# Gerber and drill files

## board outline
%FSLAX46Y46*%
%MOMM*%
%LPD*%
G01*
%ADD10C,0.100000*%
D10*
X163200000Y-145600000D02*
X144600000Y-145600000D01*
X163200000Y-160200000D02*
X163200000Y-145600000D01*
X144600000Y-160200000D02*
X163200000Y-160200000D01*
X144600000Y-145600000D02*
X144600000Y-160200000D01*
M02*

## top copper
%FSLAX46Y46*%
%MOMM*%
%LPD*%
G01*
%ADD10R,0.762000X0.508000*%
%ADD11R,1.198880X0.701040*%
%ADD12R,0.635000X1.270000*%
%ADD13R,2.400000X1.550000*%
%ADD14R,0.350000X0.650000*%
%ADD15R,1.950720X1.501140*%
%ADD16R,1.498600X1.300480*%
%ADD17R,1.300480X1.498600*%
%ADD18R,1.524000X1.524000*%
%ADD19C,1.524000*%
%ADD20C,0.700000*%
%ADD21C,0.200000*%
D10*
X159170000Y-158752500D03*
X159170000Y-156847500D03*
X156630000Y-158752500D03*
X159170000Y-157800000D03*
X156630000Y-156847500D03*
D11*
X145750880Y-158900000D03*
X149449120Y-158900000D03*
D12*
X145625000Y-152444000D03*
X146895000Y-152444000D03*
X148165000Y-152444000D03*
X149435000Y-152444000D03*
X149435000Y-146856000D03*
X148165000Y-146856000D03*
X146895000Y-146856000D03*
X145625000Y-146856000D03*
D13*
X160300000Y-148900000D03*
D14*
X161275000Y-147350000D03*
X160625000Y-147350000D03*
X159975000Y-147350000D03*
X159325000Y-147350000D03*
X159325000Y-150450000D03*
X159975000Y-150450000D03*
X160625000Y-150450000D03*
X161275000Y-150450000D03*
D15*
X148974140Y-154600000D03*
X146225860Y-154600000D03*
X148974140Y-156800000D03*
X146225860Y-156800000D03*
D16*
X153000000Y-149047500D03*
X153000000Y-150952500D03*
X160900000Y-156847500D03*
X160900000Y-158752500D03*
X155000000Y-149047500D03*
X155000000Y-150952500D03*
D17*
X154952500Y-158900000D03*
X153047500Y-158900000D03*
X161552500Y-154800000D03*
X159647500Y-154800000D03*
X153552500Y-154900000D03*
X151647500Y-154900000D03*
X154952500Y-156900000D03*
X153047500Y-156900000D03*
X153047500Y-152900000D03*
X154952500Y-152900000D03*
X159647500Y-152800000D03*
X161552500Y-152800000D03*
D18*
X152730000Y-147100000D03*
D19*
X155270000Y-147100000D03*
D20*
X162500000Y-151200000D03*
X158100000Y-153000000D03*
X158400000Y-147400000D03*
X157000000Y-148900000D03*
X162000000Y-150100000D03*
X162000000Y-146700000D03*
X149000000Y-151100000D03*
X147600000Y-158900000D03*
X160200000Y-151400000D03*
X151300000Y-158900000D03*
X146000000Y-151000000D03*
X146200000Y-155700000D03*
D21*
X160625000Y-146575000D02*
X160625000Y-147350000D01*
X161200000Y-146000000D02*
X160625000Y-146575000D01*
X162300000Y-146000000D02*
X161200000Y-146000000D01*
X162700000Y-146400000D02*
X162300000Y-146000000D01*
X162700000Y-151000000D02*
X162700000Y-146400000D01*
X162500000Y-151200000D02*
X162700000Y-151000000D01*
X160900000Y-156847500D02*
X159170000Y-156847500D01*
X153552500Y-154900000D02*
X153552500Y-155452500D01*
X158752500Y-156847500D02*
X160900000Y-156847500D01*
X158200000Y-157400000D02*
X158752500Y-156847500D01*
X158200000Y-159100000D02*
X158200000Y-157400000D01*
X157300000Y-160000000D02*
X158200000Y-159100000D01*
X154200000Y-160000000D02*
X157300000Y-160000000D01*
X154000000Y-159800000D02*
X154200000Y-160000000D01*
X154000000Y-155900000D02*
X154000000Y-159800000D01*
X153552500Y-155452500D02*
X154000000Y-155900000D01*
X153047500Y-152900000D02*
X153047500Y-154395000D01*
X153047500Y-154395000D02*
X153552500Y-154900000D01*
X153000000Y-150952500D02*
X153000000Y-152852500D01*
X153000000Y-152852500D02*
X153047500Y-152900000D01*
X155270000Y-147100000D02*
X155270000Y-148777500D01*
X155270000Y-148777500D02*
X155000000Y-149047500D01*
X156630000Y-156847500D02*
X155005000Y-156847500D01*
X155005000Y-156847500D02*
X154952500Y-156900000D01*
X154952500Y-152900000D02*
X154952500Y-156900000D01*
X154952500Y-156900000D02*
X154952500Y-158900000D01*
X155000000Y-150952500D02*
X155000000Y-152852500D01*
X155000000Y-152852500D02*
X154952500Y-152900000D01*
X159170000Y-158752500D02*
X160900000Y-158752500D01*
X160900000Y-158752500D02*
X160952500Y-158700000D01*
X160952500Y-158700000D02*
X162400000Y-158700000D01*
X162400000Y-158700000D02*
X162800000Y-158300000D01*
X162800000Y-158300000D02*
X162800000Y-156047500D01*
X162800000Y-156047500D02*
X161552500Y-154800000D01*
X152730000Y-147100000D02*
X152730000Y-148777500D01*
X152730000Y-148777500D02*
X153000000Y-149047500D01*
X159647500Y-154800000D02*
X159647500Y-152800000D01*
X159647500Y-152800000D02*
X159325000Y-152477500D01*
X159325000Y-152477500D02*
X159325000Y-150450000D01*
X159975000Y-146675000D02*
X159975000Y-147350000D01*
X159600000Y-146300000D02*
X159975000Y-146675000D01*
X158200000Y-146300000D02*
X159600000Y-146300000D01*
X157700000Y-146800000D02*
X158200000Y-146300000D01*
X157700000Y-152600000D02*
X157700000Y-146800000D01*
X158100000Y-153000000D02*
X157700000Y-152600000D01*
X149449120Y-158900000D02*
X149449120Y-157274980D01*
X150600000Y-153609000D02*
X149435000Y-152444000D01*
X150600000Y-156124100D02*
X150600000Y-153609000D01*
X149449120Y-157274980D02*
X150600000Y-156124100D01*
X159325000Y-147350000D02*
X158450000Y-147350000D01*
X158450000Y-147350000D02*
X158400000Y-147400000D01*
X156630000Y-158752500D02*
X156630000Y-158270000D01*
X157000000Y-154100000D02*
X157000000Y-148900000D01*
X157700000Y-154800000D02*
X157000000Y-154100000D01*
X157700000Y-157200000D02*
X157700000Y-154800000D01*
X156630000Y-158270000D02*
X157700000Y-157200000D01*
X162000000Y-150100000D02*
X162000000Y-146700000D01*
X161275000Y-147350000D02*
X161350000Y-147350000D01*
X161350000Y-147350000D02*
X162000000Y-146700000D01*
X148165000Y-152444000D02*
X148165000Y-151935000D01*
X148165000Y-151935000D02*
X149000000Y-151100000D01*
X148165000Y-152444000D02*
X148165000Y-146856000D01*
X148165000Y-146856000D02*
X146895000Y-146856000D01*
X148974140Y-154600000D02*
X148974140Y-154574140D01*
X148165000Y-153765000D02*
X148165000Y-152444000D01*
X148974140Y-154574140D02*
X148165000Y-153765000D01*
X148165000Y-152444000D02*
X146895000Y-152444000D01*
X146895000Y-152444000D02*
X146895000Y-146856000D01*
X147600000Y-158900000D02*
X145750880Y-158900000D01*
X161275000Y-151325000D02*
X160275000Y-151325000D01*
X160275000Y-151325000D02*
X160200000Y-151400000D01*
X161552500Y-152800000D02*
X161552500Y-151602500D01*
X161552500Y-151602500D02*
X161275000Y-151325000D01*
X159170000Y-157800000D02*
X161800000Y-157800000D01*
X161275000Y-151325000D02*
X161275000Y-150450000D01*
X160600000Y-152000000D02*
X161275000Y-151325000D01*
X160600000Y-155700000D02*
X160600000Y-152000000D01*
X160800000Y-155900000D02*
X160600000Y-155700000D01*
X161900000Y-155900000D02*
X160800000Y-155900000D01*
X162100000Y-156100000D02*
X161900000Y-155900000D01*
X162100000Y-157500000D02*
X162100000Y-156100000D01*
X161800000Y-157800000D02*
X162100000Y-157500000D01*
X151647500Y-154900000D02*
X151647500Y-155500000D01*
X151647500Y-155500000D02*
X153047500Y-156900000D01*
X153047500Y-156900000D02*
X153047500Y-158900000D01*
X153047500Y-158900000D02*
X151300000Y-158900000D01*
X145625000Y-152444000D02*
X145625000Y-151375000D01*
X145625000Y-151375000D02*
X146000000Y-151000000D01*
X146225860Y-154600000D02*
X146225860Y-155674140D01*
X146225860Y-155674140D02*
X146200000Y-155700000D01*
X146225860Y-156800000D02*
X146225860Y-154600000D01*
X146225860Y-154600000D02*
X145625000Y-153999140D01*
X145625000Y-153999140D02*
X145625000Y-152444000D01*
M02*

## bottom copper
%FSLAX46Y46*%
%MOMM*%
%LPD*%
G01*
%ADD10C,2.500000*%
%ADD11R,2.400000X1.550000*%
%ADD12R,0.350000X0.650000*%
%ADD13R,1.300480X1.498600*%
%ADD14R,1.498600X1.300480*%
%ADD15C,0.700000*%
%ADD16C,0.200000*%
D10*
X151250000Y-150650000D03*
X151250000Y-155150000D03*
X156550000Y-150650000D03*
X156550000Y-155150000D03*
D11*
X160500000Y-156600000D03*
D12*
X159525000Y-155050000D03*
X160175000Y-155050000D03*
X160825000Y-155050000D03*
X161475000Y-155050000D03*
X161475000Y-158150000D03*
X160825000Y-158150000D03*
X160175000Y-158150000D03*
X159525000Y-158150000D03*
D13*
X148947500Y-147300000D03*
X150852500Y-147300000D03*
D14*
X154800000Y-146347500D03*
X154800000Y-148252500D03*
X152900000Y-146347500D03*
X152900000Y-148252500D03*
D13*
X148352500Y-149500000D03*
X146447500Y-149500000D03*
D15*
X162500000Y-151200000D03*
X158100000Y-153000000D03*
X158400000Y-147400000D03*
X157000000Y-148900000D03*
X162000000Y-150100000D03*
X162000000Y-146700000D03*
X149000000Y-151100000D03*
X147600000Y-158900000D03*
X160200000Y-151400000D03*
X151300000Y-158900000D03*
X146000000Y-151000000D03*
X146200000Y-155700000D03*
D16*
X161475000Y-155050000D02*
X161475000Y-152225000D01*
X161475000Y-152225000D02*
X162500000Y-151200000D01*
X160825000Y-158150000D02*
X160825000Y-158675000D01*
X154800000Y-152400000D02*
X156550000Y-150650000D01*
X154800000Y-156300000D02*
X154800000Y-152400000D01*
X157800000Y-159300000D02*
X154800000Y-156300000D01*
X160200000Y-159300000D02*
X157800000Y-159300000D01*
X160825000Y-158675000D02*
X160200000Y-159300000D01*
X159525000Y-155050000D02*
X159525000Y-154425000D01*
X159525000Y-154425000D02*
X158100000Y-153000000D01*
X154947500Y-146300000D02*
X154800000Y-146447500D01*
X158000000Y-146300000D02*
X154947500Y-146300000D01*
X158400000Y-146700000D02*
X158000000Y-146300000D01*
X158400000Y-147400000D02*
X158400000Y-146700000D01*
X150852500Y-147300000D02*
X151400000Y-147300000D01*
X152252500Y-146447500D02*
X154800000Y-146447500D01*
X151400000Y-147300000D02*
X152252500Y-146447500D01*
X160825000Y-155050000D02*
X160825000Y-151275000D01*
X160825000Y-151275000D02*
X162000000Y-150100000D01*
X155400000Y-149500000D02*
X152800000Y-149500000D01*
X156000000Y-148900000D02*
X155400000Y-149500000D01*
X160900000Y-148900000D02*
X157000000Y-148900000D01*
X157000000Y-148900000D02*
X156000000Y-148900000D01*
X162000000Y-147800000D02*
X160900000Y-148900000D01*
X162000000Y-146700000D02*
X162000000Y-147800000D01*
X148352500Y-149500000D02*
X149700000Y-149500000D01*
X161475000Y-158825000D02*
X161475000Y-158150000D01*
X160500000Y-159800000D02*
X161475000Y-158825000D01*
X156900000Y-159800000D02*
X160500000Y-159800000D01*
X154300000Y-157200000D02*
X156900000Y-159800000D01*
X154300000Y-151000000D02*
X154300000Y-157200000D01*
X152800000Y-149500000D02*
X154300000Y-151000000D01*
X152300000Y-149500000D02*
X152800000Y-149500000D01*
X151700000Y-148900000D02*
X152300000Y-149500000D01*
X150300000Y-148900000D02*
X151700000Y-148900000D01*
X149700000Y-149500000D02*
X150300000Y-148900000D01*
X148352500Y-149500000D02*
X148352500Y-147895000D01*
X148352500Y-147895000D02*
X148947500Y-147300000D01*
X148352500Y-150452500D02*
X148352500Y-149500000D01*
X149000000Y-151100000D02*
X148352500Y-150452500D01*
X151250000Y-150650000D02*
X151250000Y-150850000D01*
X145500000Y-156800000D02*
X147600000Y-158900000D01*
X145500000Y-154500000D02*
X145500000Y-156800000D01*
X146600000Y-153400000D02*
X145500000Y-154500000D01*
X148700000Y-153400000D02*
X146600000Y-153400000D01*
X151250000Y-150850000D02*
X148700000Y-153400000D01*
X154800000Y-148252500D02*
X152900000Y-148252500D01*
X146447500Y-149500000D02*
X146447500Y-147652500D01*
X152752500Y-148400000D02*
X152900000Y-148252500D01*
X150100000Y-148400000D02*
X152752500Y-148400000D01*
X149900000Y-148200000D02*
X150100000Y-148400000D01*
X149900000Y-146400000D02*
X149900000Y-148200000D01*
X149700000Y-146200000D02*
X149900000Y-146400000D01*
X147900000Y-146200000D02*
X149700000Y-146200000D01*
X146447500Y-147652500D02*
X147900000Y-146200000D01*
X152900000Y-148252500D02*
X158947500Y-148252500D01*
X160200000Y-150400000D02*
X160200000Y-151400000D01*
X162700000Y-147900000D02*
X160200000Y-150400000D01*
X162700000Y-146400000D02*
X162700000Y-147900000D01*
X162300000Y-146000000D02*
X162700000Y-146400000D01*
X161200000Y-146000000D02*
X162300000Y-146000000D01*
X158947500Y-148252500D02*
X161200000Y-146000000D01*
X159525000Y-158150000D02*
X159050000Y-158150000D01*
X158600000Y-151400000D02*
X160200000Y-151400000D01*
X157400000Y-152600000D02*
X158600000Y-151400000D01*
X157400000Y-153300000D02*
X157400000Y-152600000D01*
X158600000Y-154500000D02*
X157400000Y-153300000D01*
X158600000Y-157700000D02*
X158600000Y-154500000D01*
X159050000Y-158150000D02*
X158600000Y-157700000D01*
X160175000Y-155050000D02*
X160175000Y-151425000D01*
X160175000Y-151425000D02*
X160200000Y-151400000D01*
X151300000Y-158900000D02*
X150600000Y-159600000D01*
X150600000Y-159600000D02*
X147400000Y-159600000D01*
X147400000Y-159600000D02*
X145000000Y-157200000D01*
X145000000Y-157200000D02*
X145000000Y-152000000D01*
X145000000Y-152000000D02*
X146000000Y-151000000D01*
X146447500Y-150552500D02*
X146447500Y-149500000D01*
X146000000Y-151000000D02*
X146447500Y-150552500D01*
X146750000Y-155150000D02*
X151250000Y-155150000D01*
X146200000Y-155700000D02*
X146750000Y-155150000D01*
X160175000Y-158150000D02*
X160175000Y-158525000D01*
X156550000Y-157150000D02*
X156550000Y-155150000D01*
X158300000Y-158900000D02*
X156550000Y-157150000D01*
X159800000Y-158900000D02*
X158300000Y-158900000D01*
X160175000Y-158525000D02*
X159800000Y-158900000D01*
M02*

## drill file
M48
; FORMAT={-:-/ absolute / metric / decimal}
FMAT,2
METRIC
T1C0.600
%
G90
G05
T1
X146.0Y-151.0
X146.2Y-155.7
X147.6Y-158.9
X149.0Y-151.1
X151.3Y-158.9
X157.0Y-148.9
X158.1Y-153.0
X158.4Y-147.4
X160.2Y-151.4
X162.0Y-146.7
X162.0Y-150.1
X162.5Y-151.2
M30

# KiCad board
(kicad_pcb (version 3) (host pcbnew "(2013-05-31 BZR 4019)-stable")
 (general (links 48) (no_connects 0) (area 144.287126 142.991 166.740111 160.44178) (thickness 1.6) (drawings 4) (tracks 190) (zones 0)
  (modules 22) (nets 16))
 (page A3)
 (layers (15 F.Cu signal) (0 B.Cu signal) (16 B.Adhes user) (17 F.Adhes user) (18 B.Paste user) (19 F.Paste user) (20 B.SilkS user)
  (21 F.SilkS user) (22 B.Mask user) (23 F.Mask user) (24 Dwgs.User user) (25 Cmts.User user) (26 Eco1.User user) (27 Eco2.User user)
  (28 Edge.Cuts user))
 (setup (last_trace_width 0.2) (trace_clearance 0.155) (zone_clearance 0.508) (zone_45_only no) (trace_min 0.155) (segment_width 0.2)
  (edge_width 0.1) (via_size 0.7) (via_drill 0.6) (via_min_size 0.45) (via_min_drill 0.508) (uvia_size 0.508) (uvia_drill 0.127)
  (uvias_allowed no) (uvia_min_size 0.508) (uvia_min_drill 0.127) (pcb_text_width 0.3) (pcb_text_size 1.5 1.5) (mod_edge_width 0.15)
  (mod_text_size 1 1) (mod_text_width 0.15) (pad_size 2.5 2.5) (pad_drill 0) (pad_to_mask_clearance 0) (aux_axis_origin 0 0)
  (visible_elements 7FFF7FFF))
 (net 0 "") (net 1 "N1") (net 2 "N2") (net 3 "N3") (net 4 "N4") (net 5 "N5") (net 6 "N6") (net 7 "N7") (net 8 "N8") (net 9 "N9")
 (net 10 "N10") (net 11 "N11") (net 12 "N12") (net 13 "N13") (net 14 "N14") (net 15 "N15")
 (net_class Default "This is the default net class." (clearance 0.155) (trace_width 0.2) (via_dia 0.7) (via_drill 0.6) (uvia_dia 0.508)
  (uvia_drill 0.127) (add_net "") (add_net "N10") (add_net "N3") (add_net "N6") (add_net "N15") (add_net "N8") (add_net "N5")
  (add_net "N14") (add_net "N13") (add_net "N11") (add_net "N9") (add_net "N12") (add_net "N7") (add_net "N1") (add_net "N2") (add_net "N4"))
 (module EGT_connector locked (layer B.Cu) (at 153.9 152.9)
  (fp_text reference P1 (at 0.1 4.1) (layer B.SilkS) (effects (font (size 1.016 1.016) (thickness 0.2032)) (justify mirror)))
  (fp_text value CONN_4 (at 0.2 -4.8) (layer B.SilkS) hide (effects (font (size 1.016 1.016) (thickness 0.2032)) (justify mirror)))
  (pad 1 smd circle (at -2.65 -2.25) (size 2.5 2.5) (layers B.Cu B.Paste B.Mask) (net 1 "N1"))
  (pad 2 smd circle (at -2.65 2.25) (size 2.5 2.5) (layers B.Cu B.Paste B.Mask) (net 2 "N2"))
  (pad 3 smd circle (at 2.65 -2.25) (size 2.5 2.5) (layers B.Cu B.Paste B.Mask) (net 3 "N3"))
  (pad 4 smd circle (at 2.65 2.25) (size 2.5 2.5) (layers B.Cu B.Paste B.Mask) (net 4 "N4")))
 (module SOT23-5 (layer F.Cu) (at 157.9 157.8 90)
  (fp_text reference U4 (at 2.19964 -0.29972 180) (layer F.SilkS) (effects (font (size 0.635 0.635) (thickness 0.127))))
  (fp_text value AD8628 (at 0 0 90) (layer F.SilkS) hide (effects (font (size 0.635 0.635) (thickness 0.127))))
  (pad 1 smd rect (at -0.9525 1.27 90) (size 0.508 0.762) (layers F.Cu F.Paste F.Mask) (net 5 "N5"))
  (pad 3 smd rect (at 0.9525 1.27 90) (size 0.508 0.762) (layers F.Cu F.Paste F.Mask) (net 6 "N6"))
  (pad 5 smd rect (at -0.9525 -1.27 90) (size 0.508 0.762) (layers F.Cu F.Paste F.Mask) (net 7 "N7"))
  (pad 2 smd rect (at 0 1.27 90) (size 0.508 0.762) (layers F.Cu F.Paste F.Mask) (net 2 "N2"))
  (pad 4 smd rect (at 0.9525 -1.27 90) (size 0.508 0.762) (layers F.Cu F.Paste F.Mask) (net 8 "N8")))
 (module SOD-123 (layer F.Cu) (at 147.6 158.9)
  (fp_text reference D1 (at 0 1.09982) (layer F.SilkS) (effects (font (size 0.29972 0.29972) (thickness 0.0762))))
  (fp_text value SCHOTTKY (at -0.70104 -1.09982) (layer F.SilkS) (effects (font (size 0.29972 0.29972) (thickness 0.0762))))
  (pad 1 smd rect (at -1.84912 0) (size 1.19888 0.70104) (layers F.Cu F.Paste F.Mask) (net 1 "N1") (clearance 0.14986))
  (pad 2 smd rect (at 1.84912 0) (size 1.19888 0.70104) (layers F.Cu F.Paste F.Mask) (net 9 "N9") (clearance 0.14986)))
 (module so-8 (layer F.Cu) (at 147.53 149.65)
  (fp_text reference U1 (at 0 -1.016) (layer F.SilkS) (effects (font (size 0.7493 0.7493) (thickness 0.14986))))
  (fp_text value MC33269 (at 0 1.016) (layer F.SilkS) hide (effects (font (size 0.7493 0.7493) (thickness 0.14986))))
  (pad 1 smd rect (at -1.905 2.794) (size 0.635 1.27) (layers F.Cu F.Paste F.Mask) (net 2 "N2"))
  (pad 2 smd rect (at -0.635 2.794) (size 0.635 1.27) (layers F.Cu F.Paste F.Mask) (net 7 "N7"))
  (pad 3 smd rect (at 0.635 2.794) (size 0.635 1.27) (layers F.Cu F.Paste F.Mask) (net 7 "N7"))
  (pad 4 smd rect (at 1.905 2.794) (size 0.635 1.27) (layers F.Cu F.Paste F.Mask) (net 9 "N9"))
  (pad 5 smd rect (at 1.905 -2.794) (size 0.635 1.27) (layers F.Cu F.Paste F.Mask))
  (pad 6 smd rect (at 0.635 -2.794) (size 0.635 1.27) (layers F.Cu F.Paste F.Mask) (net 7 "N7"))
  (pad 7 smd rect (at -0.635 -2.794) (size 0.635 1.27) (layers F.Cu F.Paste F.Mask) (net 7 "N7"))
  (pad 8 smd rect (at -1.905 -2.794) (size 0.635 1.27) (layers F.Cu F.Paste F.Mask)))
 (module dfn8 (layer F.Cu) (at 160.3 148.9 180)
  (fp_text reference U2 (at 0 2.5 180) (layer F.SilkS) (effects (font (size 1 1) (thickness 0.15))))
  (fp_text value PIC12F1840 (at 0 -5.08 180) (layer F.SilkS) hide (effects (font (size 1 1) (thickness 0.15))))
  (pad 9 smd rect (at 0 0 180) (size 2.4 1.55) (layers F.Cu F.Paste F.Mask))
  (pad 1 smd rect (at -0.975 1.55 180) (size 0.35 0.65) (layers F.Cu F.Paste F.Mask) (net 7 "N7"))
  (pad 2 smd rect (at -0.325 1.55 180) (size 0.35 0.65) (layers F.Cu F.Paste F.Mask) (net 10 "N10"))
  (pad 3 smd rect (at 0.325 1.55 180) (size 0.35 0.65) (layers F.Cu F.Paste F.Mask) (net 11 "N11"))
  (pad 4 smd rect (at 0.975 1.55 180) (size 0.35 0.65) (layers F.Cu F.Paste F.Mask) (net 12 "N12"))
  (pad 5 smd rect (at 0.975 -1.55 180) (size 0.35 0.65) (layers F.Cu F.Paste F.Mask) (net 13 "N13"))
  (pad 6 smd rect (at 0.325 -1.55 180) (size 0.35 0.65) (layers F.Cu F.Paste F.Mask))
  (pad 7 smd rect (at -0.325 -1.55 180) (size 0.35 0.65) (layers F.Cu F.Paste F.Mask))
  (pad 8 smd rect (at -0.975 -1.55 180) (size 0.35 0.65) (layers F.Cu F.Paste F.Mask) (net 2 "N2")))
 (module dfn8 (layer B.Cu) (at 160.5 156.6)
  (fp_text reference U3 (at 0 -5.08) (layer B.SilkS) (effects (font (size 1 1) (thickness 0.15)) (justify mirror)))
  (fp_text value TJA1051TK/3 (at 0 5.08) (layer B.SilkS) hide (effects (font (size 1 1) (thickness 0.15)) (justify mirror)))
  (pad 9 smd rect (at 0 0) (size 2.4 1.55) (layers B.Cu B.Paste B.Mask))
  (pad 1 smd rect (at -0.975 -1.55) (size 0.35 0.65) (layers B.Cu B.Paste B.Mask) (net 11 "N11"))
  (pad 2 smd rect (at -0.325 -1.55) (size 0.35 0.65) (layers B.Cu B.Paste B.Mask) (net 2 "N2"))
  (pad 3 smd rect (at 0.325 -1.55) (size 0.35 0.65) (layers B.Cu B.Paste B.Mask) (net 7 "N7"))
  (pad 4 smd rect (at 0.975 -1.55) (size 0.35 0.65) (layers B.Cu B.Paste B.Mask) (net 10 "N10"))
  (pad 5 smd rect (at 0.975 1.55) (size 0.35 0.65) (layers B.Cu B.Paste B.Mask) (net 7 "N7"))
  (pad 6 smd rect (at 0.325 1.55) (size 0.35 0.65) (layers B.Cu B.Paste B.Mask) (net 3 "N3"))
  (pad 7 smd rect (at -0.325 1.55) (size 0.35 0.65) (layers B.Cu B.Paste B.Mask) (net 4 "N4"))
  (pad 8 smd rect (at -0.975 1.55) (size 0.35 0.65) (layers B.Cu B.Paste B.Mask) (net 2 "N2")))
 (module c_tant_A (layer F.Cu) (at 147.6 154.6)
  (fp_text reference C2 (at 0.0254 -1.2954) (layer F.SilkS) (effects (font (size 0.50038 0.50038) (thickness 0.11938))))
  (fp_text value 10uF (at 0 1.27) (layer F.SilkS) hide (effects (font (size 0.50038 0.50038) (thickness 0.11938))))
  (pad 1 smd rect (at 1.37414 0) (size 1.95072 1.50114) (layers F.Cu F.Paste F.Mask) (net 7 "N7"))
  (pad 2 smd rect (at -1.37414 0) (size 1.95072 1.50114) (layers F.Cu F.Paste F.Mask) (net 2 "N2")))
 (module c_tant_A (layer F.Cu) (at 147.6 156.8)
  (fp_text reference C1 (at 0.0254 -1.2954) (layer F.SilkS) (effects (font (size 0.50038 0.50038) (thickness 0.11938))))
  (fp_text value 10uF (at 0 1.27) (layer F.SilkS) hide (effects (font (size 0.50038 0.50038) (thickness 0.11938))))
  (pad 1 smd rect (at 1.37414 0) (size 1.95072 1.50114) (layers F.Cu F.Paste F.Mask) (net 9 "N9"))
  (pad 2 smd rect (at -1.37414 0) (size 1.95072 1.50114) (layers F.Cu F.Paste F.Mask) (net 2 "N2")))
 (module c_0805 (layer F.Cu) (at 153 150 90)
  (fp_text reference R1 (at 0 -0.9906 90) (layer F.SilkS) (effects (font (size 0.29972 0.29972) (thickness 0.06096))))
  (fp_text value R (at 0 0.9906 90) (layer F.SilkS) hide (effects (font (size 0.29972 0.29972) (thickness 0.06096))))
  (pad 1 smd rect (at 0.9525 0 90) (size 1.30048 1.4986) (layers F.Cu F.Paste F.Mask) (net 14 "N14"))
  (pad 2 smd rect (at -0.9525 0 90) (size 1.30048 1.4986) (layers F.Cu F.Paste F.Mask) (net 6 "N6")))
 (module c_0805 (layer F.Cu) (at 160.9 157.8 90)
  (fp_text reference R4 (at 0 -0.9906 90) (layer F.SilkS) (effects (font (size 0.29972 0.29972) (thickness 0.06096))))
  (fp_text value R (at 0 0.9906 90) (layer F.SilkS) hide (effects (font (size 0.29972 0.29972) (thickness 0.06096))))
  (pad 1 smd rect (at 0.9525 0 90) (size 1.30048 1.4986) (layers F.Cu F.Paste F.Mask) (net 6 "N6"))
  (pad 2 smd rect (at -0.9525 0 90) (size 1.30048 1.4986) (layers F.Cu F.Paste F.Mask) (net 5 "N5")))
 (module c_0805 (layer F.Cu) (at 155 150 90)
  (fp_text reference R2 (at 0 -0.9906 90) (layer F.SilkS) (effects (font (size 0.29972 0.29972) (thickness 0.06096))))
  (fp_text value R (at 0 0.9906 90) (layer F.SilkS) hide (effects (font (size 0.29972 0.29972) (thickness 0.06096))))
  (pad 1 smd rect (at 0.9525 0 90) (size 1.30048 1.4986) (layers F.Cu F.Paste F.Mask) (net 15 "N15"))
  (pad 2 smd rect (at -0.9525 0 90) (size 1.30048 1.4986) (layers F.Cu F.Paste F.Mask) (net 8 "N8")))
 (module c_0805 (layer F.Cu) (at 154 158.9)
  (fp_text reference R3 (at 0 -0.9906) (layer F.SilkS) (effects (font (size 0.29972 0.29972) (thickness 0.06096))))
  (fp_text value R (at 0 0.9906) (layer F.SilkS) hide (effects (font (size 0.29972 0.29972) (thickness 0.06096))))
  (pad 1 smd rect (at 0.9525 0) (size 1.30048 1.4986) (layers F.Cu F.Paste F.Mask) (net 8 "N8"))
  (pad 2 smd rect (at -0.9525 0) (size 1.30048 1.4986) (layers F.Cu F.Paste F.Mask) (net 2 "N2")))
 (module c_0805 (layer B.Cu) (at 149.9 147.3 180)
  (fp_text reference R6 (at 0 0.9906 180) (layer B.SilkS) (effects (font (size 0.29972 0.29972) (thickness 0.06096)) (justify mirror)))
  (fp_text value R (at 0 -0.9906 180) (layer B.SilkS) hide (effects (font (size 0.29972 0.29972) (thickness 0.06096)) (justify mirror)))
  (pad 1 smd rect (at 0.9525 0 180) (size 1.30048 1.4986) (layers B.Cu B.Paste B.Mask) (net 7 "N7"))
  (pad 2 smd rect (at -0.9525 0 180) (size 1.30048 1.4986) (layers B.Cu B.Paste B.Mask) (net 12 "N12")))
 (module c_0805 (layer F.Cu) (at 160.6 154.8)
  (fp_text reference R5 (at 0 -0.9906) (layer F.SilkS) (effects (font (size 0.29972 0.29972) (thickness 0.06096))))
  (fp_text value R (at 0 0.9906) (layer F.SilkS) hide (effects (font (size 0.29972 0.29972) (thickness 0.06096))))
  (pad 1 smd rect (at 0.9525 0) (size 1.30048 1.4986) (layers F.Cu F.Paste F.Mask) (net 5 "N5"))
  (pad 2 smd rect (at -0.9525 0) (size 1.30048 1.4986) (layers F.Cu F.Paste F.Mask) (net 13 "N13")))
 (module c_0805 (layer F.Cu) (at 152.6 154.9)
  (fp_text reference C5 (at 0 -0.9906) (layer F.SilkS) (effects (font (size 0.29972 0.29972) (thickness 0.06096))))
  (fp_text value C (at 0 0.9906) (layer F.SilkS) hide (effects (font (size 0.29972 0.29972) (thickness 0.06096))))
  (pad 1 smd rect (at 0.9525 0) (size 1.30048 1.4986) (layers F.Cu F.Paste F.Mask) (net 6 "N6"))
  (pad 2 smd rect (at -0.9525 0) (size 1.30048 1.4986) (layers F.Cu F.Paste F.Mask) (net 2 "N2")))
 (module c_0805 (layer F.Cu) (at 154 156.9)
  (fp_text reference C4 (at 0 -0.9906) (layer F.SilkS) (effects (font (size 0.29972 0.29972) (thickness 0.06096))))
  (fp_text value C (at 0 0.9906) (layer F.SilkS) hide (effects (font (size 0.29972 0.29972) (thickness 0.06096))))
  (pad 1 smd rect (at 0.9525 0) (size 1.30048 1.4986) (layers F.Cu F.Paste F.Mask) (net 8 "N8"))
  (pad 2 smd rect (at -0.9525 0) (size 1.30048 1.4986) (layers F.Cu F.Paste F.Mask) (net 2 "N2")))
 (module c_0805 (layer F.Cu) (at 154 152.9 180)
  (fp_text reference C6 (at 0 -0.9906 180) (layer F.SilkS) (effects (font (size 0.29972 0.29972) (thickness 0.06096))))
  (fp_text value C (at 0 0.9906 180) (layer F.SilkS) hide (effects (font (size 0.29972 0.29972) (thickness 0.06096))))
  (pad 1 smd rect (at 0.9525 0 180) (size 1.30048 1.4986) (layers F.Cu F.Paste F.Mask) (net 6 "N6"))
  (pad 2 smd rect (at -0.9525 0 180) (size 1.30048 1.4986) (layers F.Cu F.Paste F.Mask) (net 8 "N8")))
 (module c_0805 (layer F.Cu) (at 160.6 152.8 180)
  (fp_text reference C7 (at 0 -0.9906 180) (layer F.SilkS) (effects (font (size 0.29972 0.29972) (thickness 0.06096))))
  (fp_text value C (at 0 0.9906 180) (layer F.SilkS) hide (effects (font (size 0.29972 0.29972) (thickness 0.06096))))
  (pad 1 smd rect (at 0.9525 0 180) (size 1.30048 1.4986) (layers F.Cu F.Paste F.Mask) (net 13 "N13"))
  (pad 2 smd rect (at -0.9525 0 180) (size 1.30048 1.4986) (layers F.Cu F.Paste F.Mask) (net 2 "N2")))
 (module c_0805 (layer B.Cu) (at 154.8 147.3 90)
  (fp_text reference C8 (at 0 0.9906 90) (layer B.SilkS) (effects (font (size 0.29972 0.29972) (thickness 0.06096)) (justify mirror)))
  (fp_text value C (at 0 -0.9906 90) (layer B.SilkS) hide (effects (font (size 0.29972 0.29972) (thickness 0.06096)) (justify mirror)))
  (pad 1 smd rect (at 0.9525 0 90) (size 1.30048 1.4986) (layers B.Cu B.Paste B.Mask) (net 12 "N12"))
  (pad 2 smd rect (at -0.9525 0 90) (size 1.30048 1.4986) (layers B.Cu B.Paste B.Mask) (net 2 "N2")))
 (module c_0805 (layer B.Cu) (at 152.9 147.3 90)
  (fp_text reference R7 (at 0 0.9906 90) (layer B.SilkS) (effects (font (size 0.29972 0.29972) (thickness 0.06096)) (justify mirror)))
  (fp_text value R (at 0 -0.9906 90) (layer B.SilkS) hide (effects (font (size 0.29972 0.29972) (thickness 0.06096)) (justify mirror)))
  (pad 1 smd rect (at 0.9525 0 90) (size 1.30048 1.4986) (layers B.Cu B.Paste B.Mask) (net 12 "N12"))
  (pad 2 smd rect (at -0.9525 0 90) (size 1.30048 1.4986) (layers B.Cu B.Paste B.Mask) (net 2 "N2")))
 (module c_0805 (layer B.Cu) (at 147.4 149.5)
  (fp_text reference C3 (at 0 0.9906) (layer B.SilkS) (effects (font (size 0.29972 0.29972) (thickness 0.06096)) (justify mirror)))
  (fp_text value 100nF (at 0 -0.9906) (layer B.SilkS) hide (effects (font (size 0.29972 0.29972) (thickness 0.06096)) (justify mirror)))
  (pad 1 smd rect (at 0.9525 0) (size 1.30048 1.4986) (layers B.Cu B.Paste B.Mask) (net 7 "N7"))
  (pad 2 smd rect (at -0.9525 0) (size 1.30048 1.4986) (layers B.Cu B.Paste B.Mask) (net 2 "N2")))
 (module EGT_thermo (layer F.Cu) (at 154 147.1)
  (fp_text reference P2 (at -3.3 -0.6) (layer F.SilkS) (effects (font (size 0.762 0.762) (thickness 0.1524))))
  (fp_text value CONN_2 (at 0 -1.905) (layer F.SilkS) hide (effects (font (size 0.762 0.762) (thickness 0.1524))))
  (pad 1 smd rect (at -1.27 0) (size 1.524 1.524) (layers F.Cu F.Paste F.Mask) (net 14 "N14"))
  (pad 2 smd circle (at 1.27 0) (size 1.524 1.524) (layers F.Cu F.Paste F.Mask) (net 15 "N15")))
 (gr_line (start 163.2 145.6) (end 144.6 145.6) (angle 90) (layer Edge.Cuts) (width 0.1))
 (gr_line (start 163.2 160.2) (end 163.2 145.6) (angle 90) (layer Edge.Cuts) (width 0.1))
 (gr_line (start 144.6 160.2) (end 163.2 160.2) (angle 90) (layer Edge.Cuts) (width 0.1))
 (gr_line (start 144.6 145.6) (end 144.6 160.2) (angle 90) (layer Edge.Cuts) (width 0.1))
 (segment (start 161.475 155.05) (end 161.475 152.225) (width 0.2) (layer B.Cu) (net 10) (status 400000))
 (segment (start 160.625 146.575) (end 160.625 147.35) (width 0.2) (layer F.Cu) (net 10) (status 800000))
 (segment (start 161.2 146) (end 160.625 146.575) (width 0.2) (layer F.Cu) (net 10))
 (segment (start 162.3 146) (end 161.2 146) (width 0.2) (layer F.Cu) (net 10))
 (segment (start 162.7 146.4) (end 162.3 146) (width 0.2) (layer F.Cu) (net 10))
 (segment (start 162.7 151) (end 162.7 146.4) (width 0.2) (layer F.Cu) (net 10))
 (segment (start 162.5 151.2) (end 162.7 151) (width 0.2) (layer F.Cu) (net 10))
 (via (at 162.5 151.2) (size 0.7) (layers F.Cu B.Cu) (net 10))
 (segment (start 161.475 152.225) (end 162.5 151.2) (width 0.2) (layer B.Cu) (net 10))
 (segment (start 160.825 158.15) (end 160.825 158.675) (width 0.2) (layer B.Cu) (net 3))
 (segment (start 154.8 152.4) (end 156.55 150.65) (width 0.2) (layer B.Cu) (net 3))
 (segment (start 154.8 156.3) (end 154.8 152.4) (width 0.2) (layer B.Cu) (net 3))
 (segment (start 157.8 159.3) (end 154.8 156.3) (width 0.2) (layer B.Cu) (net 3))
 (segment (start 160.2 159.3) (end 157.8 159.3) (width 0.2) (layer B.Cu) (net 3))
 (segment (start 160.825 158.675) (end 160.2 159.3) (width 0.2) (layer B.Cu) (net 3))
 (segment (start 160.9 156.8475) (end 159.17 156.8475) (width 0.2) (layer F.Cu) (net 6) (status C00000))
 (segment (start 153.5525 154.9) (end 153.5525 155.4525) (width 0.2) (layer F.Cu) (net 6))
 (segment (start 158.7525 156.8475) (end 160.9 156.8475) (width 0.2) (layer F.Cu) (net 6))
 (segment (start 158.2 157.4) (end 158.7525 156.8475) (width 0.2) (layer F.Cu) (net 6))
 (segment (start 158.2 159.1) (end 158.2 157.4) (width 0.2) (layer F.Cu) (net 6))
 (segment (start 157.3 160) (end 158.2 159.1) (width 0.2) (layer F.Cu) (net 6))
 (segment (start 154.2 160) (end 157.3 160) (width 0.2) (layer F.Cu) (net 6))
 (segment (start 154 159.8) (end 154.2 160) (width 0.2) (layer F.Cu) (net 6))
 (segment (start 154 155.9) (end 154 159.8) (width 0.2) (layer F.Cu) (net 6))
 (segment (start 153.5525 155.4525) (end 154 155.9) (width 0.2) (layer F.Cu) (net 6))
 (segment (start 153.0475 152.9) (end 153.0475 154.395) (width 0.2) (layer F.Cu) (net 6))
 (segment (start 153.0475 154.395) (end 153.5525 154.9) (width 0.2) (layer F.Cu) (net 6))
 (segment (start 153 150.9525) (end 153 152.8525) (width 0.2) (layer F.Cu) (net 6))
 (segment (start 153 152.8525) (end 153.0475 152.9) (width 0.2) (layer F.Cu) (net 6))
 (segment (start 155.27 147.1) (end 155.27 148.7775) (width 0.2) (layer F.Cu) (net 15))
 (segment (start 155.27 148.7775) (end 155 149.0475) (width 0.2) (layer F.Cu) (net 15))
 (segment (start 156.63 156.8475) (end 155.005 156.8475) (width 0.2) (layer F.Cu) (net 8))
 (segment (start 155.005 156.8475) (end 154.9525 156.9) (width 0.2) (layer F.Cu) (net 8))
 (segment (start 154.9525 152.9) (end 154.9525 156.9) (width 0.2) (layer F.Cu) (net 8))
 (segment (start 154.9525 156.9) (end 154.9525 158.9) (width 0.2) (layer F.Cu) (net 8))
 (segment (start 155 150.9525) (end 155 152.8525) (width 0.2) (layer F.Cu) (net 8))
 (segment (start 155 152.8525) (end 154.9525 152.9) (width 0.2) (layer F.Cu) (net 8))
 (segment (start 159.17 158.7525) (end 160.9 158.7525) (width 0.2) (layer F.Cu) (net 5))
 (segment (start 160.9 158.7525) (end 160.9525 158.7) (width 0.2) (layer F.Cu) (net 5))
 (segment (start 160.9525 158.7) (end 162.4 158.7) (width 0.2) (layer F.Cu) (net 5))
 (segment (start 162.4 158.7) (end 162.8 158.3) (width 0.2) (layer F.Cu) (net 5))
 (segment (start 162.8 158.3) (end 162.8 156.0475) (width 0.2) (layer F.Cu) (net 5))
 (segment (start 162.8 156.0475) (end 161.5525 154.8) (width 0.2) (layer F.Cu) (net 5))
 (segment (start 152.73 147.1) (end 152.73 148.7775) (width 0.2) (layer F.Cu) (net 14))
 (segment (start 152.73 148.7775) (end 153 149.0475) (width 0.2) (layer F.Cu) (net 14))
 (segment (start 159.6475 154.8) (end 159.6475 152.8) (width 0.2) (layer F.Cu) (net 13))
 (segment (start 159.6475 152.8) (end 159.325 152.4775) (width 0.2) (layer F.Cu) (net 13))
 (segment (start 159.325 152.4775) (end 159.325 150.45) (width 0.2) (layer F.Cu) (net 13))
 (segment (start 159.525 155.05) (end 159.525 154.425) (width 0.2) (layer B.Cu) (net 11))
 (segment (start 159.975 146.675) (end 159.975 147.35) (width 0.2) (layer F.Cu) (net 11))
 (segment (start 159.6 146.3) (end 159.975 146.675) (width 0.2) (layer F.Cu) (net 11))
 (segment (start 158.2 146.3) (end 159.6 146.3) (width 0.2) (layer F.Cu) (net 11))
 (segment (start 157.7 146.8) (end 158.2 146.3) (width 0.2) (layer F.Cu) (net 11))
 (segment (start 157.7 152.6) (end 157.7 146.8) (width 0.2) (layer F.Cu) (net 11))
 (segment (start 158.1 153) (end 157.7 152.6) (width 0.2) (layer F.Cu) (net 11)) (via (at 158.1 153) (size 0.7) (layers F.Cu B.Cu) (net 11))
 (segment (start 159.525 154.425) (end 158.1 153) (width 0.2) (layer B.Cu) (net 11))
 (segment (start 149.44912 158.9) (end 149.44912 157.27498) (width 0.2) (layer F.Cu) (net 9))
 (segment (start 150.6 153.609) (end 149.435 152.444) (width 0.2) (layer F.Cu) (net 9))
 (segment (start 150.6 156.1241) (end 150.6 153.609) (width 0.2) (layer F.Cu) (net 9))
 (segment (start 149.44912 157.27498) (end 150.6 156.1241) (width 0.2) (layer F.Cu) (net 9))
 (segment (start 159.325 147.35) (end 158.45 147.35) (width 0.2) (layer F.Cu) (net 12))
 (segment (start 154.9475 146.3) (end 154.8 146.4475) (width 0.2) (layer B.Cu) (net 12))
 (segment (start 158 146.3) (end 154.9475 146.3) (width 0.2) (layer B.Cu) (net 12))
 (segment (start 158.4 146.7) (end 158 146.3) (width 0.2) (layer B.Cu) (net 12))
 (segment (start 158.4 147.4) (end 158.4 146.7) (width 0.2) (layer B.Cu) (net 12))
 (via (at 158.4 147.4) (size 0.7) (layers F.Cu B.Cu) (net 12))
 (segment (start 158.45 147.35) (end 158.4 147.4) (width 0.2) (layer F.Cu) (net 12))
 (segment (start 150.8525 147.3) (end 151.4 147.3) (width 0.2) (layer B.Cu) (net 12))
 (segment (start 152.2525 146.4475) (end 154.8 146.4475) (width 0.2) (layer B.Cu) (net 12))
 (segment (start 151.4 147.3) (end 152.2525 146.4475) (width 0.2) (layer B.Cu) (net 12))
 (segment (start 156.63 158.7525) (end 156.63 158.27) (width 0.2) (layer F.Cu) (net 7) (status 400000))
 (via (at 157 148.9) (size 0.7) (layers F.Cu B.Cu) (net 7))
 (segment (start 157 154.1) (end 157 148.9) (width 0.2) (layer F.Cu) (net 7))
 (segment (start 157.7 154.8) (end 157 154.1) (width 0.2) (layer F.Cu) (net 7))
 (segment (start 157.7 157.2) (end 157.7 154.8) (width 0.2) (layer F.Cu) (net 7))
 (segment (start 156.63 158.27) (end 157.7 157.2) (width 0.2) (layer F.Cu) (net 7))
 (segment (start 160.825 155.05) (end 160.825 151.275) (width 0.2) (layer B.Cu) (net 7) (status 400000))
 (segment (start 162 150.1) (end 162 146.7) (width 0.2) (layer F.Cu) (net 7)) (via (at 162 150.1) (size 0.7) (layers F.Cu B.Cu) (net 7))
 (segment (start 160.825 151.275) (end 162 150.1) (width 0.2) (layer B.Cu) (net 7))
 (segment (start 161.275 147.35) (end 161.35 147.35) (width 0.2) (layer F.Cu) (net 7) (status C00000))
 (segment (start 155.4 149.5) (end 152.8 149.5) (width 0.2) (layer B.Cu) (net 7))
 (segment (start 156 148.9) (end 155.4 149.5) (width 0.2) (layer B.Cu) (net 7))
 (segment (start 160.9 148.9) (end 157 148.9) (width 0.2) (layer B.Cu) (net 7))
 (segment (start 157 148.9) (end 156 148.9) (width 0.2) (layer B.Cu) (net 7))
 (segment (start 162 147.8) (end 160.9 148.9) (width 0.2) (layer B.Cu) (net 7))
 (segment (start 162 146.7) (end 162 147.8) (width 0.2) (layer B.Cu) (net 7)) (via (at 162 146.7) (size 0.7) (layers F.Cu B.Cu) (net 7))
 (segment (start 161.35 147.35) (end 162 146.7) (width 0.2) (layer F.Cu) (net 7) (status 400000))
 (segment (start 148.3525 149.5) (end 149.7 149.5) (width 0.2) (layer B.Cu) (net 7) (status 400000))
 (segment (start 161.475 158.825) (end 161.475 158.15) (width 0.2) (layer B.Cu) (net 7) (status 800000))
 (segment (start 160.5 159.8) (end 161.475 158.825) (width 0.2) (layer B.Cu) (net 7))
 (segment (start 156.9 159.8) (end 160.5 159.8) (width 0.2) (layer B.Cu) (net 7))
 (segment (start 154.3 157.2) (end 156.9 159.8) (width 0.2) (layer B.Cu) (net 7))
 (segment (start 154.3 151) (end 154.3 157.2) (width 0.2) (layer B.Cu) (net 7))
 (segment (start 152.8 149.5) (end 154.3 151) (width 0.2) (layer B.Cu) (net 7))
 (segment (start 152.3 149.5) (end 152.8 149.5) (width 0.2) (layer B.Cu) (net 7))
 (segment (start 151.7 148.9) (end 152.3 149.5) (width 0.2) (layer B.Cu) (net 7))
 (segment (start 150.3 148.9) (end 151.7 148.9) (width 0.2) (layer B.Cu) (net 7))
 (segment (start 149.7 149.5) (end 150.3 148.9) (width 0.2) (layer B.Cu) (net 7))
 (segment (start 148.3525 149.5) (end 148.3525 147.895) (width 0.2) (layer B.Cu) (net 7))
 (segment (start 148.3525 147.895) (end 148.9475 147.3) (width 0.2) (layer B.Cu) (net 7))
 (segment (start 148.165 152.444) (end 148.165 151.935) (width 0.2) (layer F.Cu) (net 7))
 (segment (start 148.3525 150.4525) (end 148.3525 149.5) (width 0.2) (layer B.Cu) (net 7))
 (segment (start 149 151.1) (end 148.3525 150.4525) (width 0.2) (layer B.Cu) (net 7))
 (via (at 149 151.1) (size 0.7) (layers F.Cu B.Cu) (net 7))
 (segment (start 148.165 151.935) (end 149 151.1) (width 0.2) (layer F.Cu) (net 7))
 (segment (start 148.165 152.444) (end 148.165 146.856) (width 0.2) (layer F.Cu) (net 7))
 (segment (start 148.165 146.856) (end 146.895 146.856) (width 0.2) (layer F.Cu) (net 7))
 (segment (start 148.97414 154.6) (end 148.97414 154.57414) (width 0.2) (layer F.Cu) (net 7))
 (segment (start 148.165 153.765) (end 148.165 152.444) (width 0.2) (layer F.Cu) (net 7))
 (segment (start 148.97414 154.57414) (end 148.165 153.765) (width 0.2) (layer F.Cu) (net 7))
 (segment (start 148.165 152.444) (end 146.895 152.444) (width 0.2) (layer F.Cu) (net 7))
 (segment (start 146.895 152.444) (end 146.895 146.856) (width 0.2) (layer F.Cu) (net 7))
 (segment (start 151.25 150.65) (end 151.25 150.85) (width 0.2) (layer B.Cu) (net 1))
 (segment (start 147.6 158.9) (end 145.75088 158.9) (width 0.2) (layer F.Cu) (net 1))
 (via (at 147.6 158.9) (size 0.7) (layers F.Cu B.Cu) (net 1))
 (segment (start 145.5 156.8) (end 147.6 158.9) (width 0.2) (layer B.Cu) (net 1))
 (segment (start 145.5 154.5) (end 145.5 156.8) (width 0.2) (layer B.Cu) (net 1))
 (segment (start 146.6 153.4) (end 145.5 154.5) (width 0.2) (layer B.Cu) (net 1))
 (segment (start 148.7 153.4) (end 146.6 153.4) (width 0.2) (layer B.Cu) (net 1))
 (segment (start 151.25 150.85) (end 148.7 153.4) (width 0.2) (layer B.Cu) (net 1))
 (segment (start 154.8 148.2525) (end 152.9 148.2525) (width 0.2) (layer B.Cu) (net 2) (status C00000))
 (segment (start 146.4475 149.5) (end 146.4475 147.6525) (width 0.2) (layer B.Cu) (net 2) (status 400000))
 (segment (start 152.7525 148.4) (end 152.9 148.2525) (width 0.2) (layer B.Cu) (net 2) (status C00000))
 (segment (start 150.1 148.4) (end 152.7525 148.4) (width 0.2) (layer B.Cu) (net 2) (status 800000))
 (segment (start 149.9 148.2) (end 150.1 148.4) (width 0.2) (layer B.Cu) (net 2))
 (segment (start 149.9 146.4) (end 149.9 148.2) (width 0.2) (layer B.Cu) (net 2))
 (segment (start 149.7 146.2) (end 149.9 146.4) (width 0.2) (layer B.Cu) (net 2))
 (segment (start 147.9 146.2) (end 149.7 146.2) (width 0.2) (layer B.Cu) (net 2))
 (segment (start 146.4475 147.6525) (end 147.9 146.2) (width 0.2) (layer B.Cu) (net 2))
 (segment (start 152.9 148.2525) (end 158.9475 148.2525) (width 0.2) (layer B.Cu) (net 2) (status 400000))
 (segment (start 160.2 150.4) (end 160.2 151.4) (width 0.2) (layer B.Cu) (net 2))
 (segment (start 162.7 147.9) (end 160.2 150.4) (width 0.2) (layer B.Cu) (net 2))
 (segment (start 162.7 146.4) (end 162.7 147.9) (width 0.2) (layer B.Cu) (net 2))
 (segment (start 162.3 146) (end 162.7 146.4) (width 0.2) (layer B.Cu) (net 2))
 (segment (start 161.2 146) (end 162.3 146) (width 0.2) (layer B.Cu) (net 2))
 (segment (start 158.9475 148.2525) (end 161.2 146) (width 0.2) (layer B.Cu) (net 2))
 (segment (start 159.525 158.15) (end 159.05 158.15) (width 0.2) (layer B.Cu) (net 2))
 (segment (start 158.6 151.4) (end 160.2 151.4) (width 0.2) (layer B.Cu) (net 2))
 (segment (start 157.4 152.6) (end 158.6 151.4) (width 0.2) (layer B.Cu) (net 2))
 (segment (start 157.4 153.3) (end 157.4 152.6) (width 0.2) (layer B.Cu) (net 2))
 (segment (start 158.6 154.5) (end 157.4 153.3) (width 0.2) (layer B.Cu) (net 2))
 (segment (start 158.6 157.7) (end 158.6 154.5) (width 0.2) (layer B.Cu) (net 2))
 (segment (start 159.05 158.15) (end 158.6 157.7) (width 0.2) (layer B.Cu) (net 2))
 (segment (start 160.175 155.05) (end 160.175 151.425) (width 0.2) (layer B.Cu) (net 2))
 (segment (start 160.175 151.425) (end 160.2 151.4) (width 0.2) (layer B.Cu) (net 2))
 (segment (start 161.275 151.325) (end 160.275 151.325) (width 0.2) (layer F.Cu) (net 2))
 (via (at 160.2 151.4) (size 0.7) (layers F.Cu B.Cu) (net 2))
 (segment (start 160.275 151.325) (end 160.2 151.4) (width 0.2) (layer F.Cu) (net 2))
 (segment (start 161.5525 152.8) (end 161.5525 151.6025) (width 0.2) (layer F.Cu) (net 2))
 (segment (start 161.5525 151.6025) (end 161.275 151.325) (width 0.2) (layer F.Cu) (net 2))
 (segment (start 159.17 157.8) (end 161.8 157.8) (width 0.2) (layer F.Cu) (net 2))
 (segment (start 161.275 151.325) (end 161.275 150.45) (width 0.2) (layer F.Cu) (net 2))
 (segment (start 160.6 152) (end 161.275 151.325) (width 0.2) (layer F.Cu) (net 2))
 (segment (start 160.6 155.7) (end 160.6 152) (width 0.2) (layer F.Cu) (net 2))
 (segment (start 160.8 155.9) (end 160.6 155.7) (width 0.2) (layer F.Cu) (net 2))
 (segment (start 161.9 155.9) (end 160.8 155.9) (width 0.2) (layer F.Cu) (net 2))
 (segment (start 162.1 156.1) (end 161.9 155.9) (width 0.2) (layer F.Cu) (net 2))
 (segment (start 162.1 157.5) (end 162.1 156.1) (width 0.2) (layer F.Cu) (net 2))
 (segment (start 161.8 157.8) (end 162.1 157.5) (width 0.2) (layer F.Cu) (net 2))
 (segment (start 151.6475 154.9) (end 151.6475 155.5) (width 0.2) (layer F.Cu) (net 2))
 (segment (start 151.6475 155.5) (end 153.0475 156.9) (width 0.2) (layer F.Cu) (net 2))
 (segment (start 153.0475 156.9) (end 153.0475 158.9) (width 0.2) (layer F.Cu) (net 2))
 (segment (start 153.0475 158.9) (end 151.3 158.9) (width 0.2) (layer F.Cu) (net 2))
 (via (at 151.3 158.9) (size 0.7) (layers F.Cu B.Cu) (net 2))
 (segment (start 151.3 158.9) (end 150.6 159.6) (width 0.2) (layer B.Cu) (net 2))
 (segment (start 150.6 159.6) (end 147.4 159.6) (width 0.2) (layer B.Cu) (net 2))
 (segment (start 147.4 159.6) (end 145 157.2) (width 0.2) (layer B.Cu) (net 2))
 (segment (start 145 157.2) (end 145 152) (width 0.2) (layer B.Cu) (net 2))
 (segment (start 145 152) (end 146 151) (width 0.2) (layer B.Cu) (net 2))
 (segment (start 145.625 152.444) (end 145.625 151.375) (width 0.2) (layer F.Cu) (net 2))
 (segment (start 146.4475 150.5525) (end 146.4475 149.5) (width 0.2) (layer B.Cu) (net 2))
 (segment (start 146 151) (end 146.4475 150.5525) (width 0.2) (layer B.Cu) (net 2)) (via (at 146 151) (size 0.7) (layers F.Cu B.Cu) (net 2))
 (segment (start 145.625 151.375) (end 146 151) (width 0.2) (layer F.Cu) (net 2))
 (segment (start 146.22586 154.6) (end 146.22586 155.67414) (width 0.2) (layer F.Cu) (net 2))
 (segment (start 146.75 155.15) (end 151.25 155.15) (width 0.2) (layer B.Cu) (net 2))
 (segment (start 146.2 155.7) (end 146.75 155.15) (width 0.2) (layer B.Cu) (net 2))
 (via (at 146.2 155.7) (size 0.7) (layers F.Cu B.Cu) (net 2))
 (segment (start 146.22586 155.67414) (end 146.2 155.7) (width 0.2) (layer F.Cu) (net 2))
 (segment (start 146.22586 156.8) (end 146.22586 154.6) (width 0.2) (layer F.Cu) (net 2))
 (segment (start 146.22586 154.6) (end 145.625 153.99914) (width 0.2) (layer F.Cu) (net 2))
 (segment (start 145.625 153.99914) (end 145.625 152.444) (width 0.2) (layer F.Cu) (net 2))
 (segment (start 160.175 158.15) (end 160.175 158.525) (width 0.2) (layer B.Cu) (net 4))
 (segment (start 156.55 157.15) (end 156.55 155.15) (width 0.2) (layer B.Cu) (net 4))
 (segment (start 158.3 158.9) (end 156.55 157.15) (width 0.2) (layer B.Cu) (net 4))
 (segment (start 159.8 158.9) (end 158.3 158.9) (width 0.2) (layer B.Cu) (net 4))
 (segment (start 160.175 158.525) (end 159.8 158.9) (width 0.2) (layer B.Cu) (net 4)))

